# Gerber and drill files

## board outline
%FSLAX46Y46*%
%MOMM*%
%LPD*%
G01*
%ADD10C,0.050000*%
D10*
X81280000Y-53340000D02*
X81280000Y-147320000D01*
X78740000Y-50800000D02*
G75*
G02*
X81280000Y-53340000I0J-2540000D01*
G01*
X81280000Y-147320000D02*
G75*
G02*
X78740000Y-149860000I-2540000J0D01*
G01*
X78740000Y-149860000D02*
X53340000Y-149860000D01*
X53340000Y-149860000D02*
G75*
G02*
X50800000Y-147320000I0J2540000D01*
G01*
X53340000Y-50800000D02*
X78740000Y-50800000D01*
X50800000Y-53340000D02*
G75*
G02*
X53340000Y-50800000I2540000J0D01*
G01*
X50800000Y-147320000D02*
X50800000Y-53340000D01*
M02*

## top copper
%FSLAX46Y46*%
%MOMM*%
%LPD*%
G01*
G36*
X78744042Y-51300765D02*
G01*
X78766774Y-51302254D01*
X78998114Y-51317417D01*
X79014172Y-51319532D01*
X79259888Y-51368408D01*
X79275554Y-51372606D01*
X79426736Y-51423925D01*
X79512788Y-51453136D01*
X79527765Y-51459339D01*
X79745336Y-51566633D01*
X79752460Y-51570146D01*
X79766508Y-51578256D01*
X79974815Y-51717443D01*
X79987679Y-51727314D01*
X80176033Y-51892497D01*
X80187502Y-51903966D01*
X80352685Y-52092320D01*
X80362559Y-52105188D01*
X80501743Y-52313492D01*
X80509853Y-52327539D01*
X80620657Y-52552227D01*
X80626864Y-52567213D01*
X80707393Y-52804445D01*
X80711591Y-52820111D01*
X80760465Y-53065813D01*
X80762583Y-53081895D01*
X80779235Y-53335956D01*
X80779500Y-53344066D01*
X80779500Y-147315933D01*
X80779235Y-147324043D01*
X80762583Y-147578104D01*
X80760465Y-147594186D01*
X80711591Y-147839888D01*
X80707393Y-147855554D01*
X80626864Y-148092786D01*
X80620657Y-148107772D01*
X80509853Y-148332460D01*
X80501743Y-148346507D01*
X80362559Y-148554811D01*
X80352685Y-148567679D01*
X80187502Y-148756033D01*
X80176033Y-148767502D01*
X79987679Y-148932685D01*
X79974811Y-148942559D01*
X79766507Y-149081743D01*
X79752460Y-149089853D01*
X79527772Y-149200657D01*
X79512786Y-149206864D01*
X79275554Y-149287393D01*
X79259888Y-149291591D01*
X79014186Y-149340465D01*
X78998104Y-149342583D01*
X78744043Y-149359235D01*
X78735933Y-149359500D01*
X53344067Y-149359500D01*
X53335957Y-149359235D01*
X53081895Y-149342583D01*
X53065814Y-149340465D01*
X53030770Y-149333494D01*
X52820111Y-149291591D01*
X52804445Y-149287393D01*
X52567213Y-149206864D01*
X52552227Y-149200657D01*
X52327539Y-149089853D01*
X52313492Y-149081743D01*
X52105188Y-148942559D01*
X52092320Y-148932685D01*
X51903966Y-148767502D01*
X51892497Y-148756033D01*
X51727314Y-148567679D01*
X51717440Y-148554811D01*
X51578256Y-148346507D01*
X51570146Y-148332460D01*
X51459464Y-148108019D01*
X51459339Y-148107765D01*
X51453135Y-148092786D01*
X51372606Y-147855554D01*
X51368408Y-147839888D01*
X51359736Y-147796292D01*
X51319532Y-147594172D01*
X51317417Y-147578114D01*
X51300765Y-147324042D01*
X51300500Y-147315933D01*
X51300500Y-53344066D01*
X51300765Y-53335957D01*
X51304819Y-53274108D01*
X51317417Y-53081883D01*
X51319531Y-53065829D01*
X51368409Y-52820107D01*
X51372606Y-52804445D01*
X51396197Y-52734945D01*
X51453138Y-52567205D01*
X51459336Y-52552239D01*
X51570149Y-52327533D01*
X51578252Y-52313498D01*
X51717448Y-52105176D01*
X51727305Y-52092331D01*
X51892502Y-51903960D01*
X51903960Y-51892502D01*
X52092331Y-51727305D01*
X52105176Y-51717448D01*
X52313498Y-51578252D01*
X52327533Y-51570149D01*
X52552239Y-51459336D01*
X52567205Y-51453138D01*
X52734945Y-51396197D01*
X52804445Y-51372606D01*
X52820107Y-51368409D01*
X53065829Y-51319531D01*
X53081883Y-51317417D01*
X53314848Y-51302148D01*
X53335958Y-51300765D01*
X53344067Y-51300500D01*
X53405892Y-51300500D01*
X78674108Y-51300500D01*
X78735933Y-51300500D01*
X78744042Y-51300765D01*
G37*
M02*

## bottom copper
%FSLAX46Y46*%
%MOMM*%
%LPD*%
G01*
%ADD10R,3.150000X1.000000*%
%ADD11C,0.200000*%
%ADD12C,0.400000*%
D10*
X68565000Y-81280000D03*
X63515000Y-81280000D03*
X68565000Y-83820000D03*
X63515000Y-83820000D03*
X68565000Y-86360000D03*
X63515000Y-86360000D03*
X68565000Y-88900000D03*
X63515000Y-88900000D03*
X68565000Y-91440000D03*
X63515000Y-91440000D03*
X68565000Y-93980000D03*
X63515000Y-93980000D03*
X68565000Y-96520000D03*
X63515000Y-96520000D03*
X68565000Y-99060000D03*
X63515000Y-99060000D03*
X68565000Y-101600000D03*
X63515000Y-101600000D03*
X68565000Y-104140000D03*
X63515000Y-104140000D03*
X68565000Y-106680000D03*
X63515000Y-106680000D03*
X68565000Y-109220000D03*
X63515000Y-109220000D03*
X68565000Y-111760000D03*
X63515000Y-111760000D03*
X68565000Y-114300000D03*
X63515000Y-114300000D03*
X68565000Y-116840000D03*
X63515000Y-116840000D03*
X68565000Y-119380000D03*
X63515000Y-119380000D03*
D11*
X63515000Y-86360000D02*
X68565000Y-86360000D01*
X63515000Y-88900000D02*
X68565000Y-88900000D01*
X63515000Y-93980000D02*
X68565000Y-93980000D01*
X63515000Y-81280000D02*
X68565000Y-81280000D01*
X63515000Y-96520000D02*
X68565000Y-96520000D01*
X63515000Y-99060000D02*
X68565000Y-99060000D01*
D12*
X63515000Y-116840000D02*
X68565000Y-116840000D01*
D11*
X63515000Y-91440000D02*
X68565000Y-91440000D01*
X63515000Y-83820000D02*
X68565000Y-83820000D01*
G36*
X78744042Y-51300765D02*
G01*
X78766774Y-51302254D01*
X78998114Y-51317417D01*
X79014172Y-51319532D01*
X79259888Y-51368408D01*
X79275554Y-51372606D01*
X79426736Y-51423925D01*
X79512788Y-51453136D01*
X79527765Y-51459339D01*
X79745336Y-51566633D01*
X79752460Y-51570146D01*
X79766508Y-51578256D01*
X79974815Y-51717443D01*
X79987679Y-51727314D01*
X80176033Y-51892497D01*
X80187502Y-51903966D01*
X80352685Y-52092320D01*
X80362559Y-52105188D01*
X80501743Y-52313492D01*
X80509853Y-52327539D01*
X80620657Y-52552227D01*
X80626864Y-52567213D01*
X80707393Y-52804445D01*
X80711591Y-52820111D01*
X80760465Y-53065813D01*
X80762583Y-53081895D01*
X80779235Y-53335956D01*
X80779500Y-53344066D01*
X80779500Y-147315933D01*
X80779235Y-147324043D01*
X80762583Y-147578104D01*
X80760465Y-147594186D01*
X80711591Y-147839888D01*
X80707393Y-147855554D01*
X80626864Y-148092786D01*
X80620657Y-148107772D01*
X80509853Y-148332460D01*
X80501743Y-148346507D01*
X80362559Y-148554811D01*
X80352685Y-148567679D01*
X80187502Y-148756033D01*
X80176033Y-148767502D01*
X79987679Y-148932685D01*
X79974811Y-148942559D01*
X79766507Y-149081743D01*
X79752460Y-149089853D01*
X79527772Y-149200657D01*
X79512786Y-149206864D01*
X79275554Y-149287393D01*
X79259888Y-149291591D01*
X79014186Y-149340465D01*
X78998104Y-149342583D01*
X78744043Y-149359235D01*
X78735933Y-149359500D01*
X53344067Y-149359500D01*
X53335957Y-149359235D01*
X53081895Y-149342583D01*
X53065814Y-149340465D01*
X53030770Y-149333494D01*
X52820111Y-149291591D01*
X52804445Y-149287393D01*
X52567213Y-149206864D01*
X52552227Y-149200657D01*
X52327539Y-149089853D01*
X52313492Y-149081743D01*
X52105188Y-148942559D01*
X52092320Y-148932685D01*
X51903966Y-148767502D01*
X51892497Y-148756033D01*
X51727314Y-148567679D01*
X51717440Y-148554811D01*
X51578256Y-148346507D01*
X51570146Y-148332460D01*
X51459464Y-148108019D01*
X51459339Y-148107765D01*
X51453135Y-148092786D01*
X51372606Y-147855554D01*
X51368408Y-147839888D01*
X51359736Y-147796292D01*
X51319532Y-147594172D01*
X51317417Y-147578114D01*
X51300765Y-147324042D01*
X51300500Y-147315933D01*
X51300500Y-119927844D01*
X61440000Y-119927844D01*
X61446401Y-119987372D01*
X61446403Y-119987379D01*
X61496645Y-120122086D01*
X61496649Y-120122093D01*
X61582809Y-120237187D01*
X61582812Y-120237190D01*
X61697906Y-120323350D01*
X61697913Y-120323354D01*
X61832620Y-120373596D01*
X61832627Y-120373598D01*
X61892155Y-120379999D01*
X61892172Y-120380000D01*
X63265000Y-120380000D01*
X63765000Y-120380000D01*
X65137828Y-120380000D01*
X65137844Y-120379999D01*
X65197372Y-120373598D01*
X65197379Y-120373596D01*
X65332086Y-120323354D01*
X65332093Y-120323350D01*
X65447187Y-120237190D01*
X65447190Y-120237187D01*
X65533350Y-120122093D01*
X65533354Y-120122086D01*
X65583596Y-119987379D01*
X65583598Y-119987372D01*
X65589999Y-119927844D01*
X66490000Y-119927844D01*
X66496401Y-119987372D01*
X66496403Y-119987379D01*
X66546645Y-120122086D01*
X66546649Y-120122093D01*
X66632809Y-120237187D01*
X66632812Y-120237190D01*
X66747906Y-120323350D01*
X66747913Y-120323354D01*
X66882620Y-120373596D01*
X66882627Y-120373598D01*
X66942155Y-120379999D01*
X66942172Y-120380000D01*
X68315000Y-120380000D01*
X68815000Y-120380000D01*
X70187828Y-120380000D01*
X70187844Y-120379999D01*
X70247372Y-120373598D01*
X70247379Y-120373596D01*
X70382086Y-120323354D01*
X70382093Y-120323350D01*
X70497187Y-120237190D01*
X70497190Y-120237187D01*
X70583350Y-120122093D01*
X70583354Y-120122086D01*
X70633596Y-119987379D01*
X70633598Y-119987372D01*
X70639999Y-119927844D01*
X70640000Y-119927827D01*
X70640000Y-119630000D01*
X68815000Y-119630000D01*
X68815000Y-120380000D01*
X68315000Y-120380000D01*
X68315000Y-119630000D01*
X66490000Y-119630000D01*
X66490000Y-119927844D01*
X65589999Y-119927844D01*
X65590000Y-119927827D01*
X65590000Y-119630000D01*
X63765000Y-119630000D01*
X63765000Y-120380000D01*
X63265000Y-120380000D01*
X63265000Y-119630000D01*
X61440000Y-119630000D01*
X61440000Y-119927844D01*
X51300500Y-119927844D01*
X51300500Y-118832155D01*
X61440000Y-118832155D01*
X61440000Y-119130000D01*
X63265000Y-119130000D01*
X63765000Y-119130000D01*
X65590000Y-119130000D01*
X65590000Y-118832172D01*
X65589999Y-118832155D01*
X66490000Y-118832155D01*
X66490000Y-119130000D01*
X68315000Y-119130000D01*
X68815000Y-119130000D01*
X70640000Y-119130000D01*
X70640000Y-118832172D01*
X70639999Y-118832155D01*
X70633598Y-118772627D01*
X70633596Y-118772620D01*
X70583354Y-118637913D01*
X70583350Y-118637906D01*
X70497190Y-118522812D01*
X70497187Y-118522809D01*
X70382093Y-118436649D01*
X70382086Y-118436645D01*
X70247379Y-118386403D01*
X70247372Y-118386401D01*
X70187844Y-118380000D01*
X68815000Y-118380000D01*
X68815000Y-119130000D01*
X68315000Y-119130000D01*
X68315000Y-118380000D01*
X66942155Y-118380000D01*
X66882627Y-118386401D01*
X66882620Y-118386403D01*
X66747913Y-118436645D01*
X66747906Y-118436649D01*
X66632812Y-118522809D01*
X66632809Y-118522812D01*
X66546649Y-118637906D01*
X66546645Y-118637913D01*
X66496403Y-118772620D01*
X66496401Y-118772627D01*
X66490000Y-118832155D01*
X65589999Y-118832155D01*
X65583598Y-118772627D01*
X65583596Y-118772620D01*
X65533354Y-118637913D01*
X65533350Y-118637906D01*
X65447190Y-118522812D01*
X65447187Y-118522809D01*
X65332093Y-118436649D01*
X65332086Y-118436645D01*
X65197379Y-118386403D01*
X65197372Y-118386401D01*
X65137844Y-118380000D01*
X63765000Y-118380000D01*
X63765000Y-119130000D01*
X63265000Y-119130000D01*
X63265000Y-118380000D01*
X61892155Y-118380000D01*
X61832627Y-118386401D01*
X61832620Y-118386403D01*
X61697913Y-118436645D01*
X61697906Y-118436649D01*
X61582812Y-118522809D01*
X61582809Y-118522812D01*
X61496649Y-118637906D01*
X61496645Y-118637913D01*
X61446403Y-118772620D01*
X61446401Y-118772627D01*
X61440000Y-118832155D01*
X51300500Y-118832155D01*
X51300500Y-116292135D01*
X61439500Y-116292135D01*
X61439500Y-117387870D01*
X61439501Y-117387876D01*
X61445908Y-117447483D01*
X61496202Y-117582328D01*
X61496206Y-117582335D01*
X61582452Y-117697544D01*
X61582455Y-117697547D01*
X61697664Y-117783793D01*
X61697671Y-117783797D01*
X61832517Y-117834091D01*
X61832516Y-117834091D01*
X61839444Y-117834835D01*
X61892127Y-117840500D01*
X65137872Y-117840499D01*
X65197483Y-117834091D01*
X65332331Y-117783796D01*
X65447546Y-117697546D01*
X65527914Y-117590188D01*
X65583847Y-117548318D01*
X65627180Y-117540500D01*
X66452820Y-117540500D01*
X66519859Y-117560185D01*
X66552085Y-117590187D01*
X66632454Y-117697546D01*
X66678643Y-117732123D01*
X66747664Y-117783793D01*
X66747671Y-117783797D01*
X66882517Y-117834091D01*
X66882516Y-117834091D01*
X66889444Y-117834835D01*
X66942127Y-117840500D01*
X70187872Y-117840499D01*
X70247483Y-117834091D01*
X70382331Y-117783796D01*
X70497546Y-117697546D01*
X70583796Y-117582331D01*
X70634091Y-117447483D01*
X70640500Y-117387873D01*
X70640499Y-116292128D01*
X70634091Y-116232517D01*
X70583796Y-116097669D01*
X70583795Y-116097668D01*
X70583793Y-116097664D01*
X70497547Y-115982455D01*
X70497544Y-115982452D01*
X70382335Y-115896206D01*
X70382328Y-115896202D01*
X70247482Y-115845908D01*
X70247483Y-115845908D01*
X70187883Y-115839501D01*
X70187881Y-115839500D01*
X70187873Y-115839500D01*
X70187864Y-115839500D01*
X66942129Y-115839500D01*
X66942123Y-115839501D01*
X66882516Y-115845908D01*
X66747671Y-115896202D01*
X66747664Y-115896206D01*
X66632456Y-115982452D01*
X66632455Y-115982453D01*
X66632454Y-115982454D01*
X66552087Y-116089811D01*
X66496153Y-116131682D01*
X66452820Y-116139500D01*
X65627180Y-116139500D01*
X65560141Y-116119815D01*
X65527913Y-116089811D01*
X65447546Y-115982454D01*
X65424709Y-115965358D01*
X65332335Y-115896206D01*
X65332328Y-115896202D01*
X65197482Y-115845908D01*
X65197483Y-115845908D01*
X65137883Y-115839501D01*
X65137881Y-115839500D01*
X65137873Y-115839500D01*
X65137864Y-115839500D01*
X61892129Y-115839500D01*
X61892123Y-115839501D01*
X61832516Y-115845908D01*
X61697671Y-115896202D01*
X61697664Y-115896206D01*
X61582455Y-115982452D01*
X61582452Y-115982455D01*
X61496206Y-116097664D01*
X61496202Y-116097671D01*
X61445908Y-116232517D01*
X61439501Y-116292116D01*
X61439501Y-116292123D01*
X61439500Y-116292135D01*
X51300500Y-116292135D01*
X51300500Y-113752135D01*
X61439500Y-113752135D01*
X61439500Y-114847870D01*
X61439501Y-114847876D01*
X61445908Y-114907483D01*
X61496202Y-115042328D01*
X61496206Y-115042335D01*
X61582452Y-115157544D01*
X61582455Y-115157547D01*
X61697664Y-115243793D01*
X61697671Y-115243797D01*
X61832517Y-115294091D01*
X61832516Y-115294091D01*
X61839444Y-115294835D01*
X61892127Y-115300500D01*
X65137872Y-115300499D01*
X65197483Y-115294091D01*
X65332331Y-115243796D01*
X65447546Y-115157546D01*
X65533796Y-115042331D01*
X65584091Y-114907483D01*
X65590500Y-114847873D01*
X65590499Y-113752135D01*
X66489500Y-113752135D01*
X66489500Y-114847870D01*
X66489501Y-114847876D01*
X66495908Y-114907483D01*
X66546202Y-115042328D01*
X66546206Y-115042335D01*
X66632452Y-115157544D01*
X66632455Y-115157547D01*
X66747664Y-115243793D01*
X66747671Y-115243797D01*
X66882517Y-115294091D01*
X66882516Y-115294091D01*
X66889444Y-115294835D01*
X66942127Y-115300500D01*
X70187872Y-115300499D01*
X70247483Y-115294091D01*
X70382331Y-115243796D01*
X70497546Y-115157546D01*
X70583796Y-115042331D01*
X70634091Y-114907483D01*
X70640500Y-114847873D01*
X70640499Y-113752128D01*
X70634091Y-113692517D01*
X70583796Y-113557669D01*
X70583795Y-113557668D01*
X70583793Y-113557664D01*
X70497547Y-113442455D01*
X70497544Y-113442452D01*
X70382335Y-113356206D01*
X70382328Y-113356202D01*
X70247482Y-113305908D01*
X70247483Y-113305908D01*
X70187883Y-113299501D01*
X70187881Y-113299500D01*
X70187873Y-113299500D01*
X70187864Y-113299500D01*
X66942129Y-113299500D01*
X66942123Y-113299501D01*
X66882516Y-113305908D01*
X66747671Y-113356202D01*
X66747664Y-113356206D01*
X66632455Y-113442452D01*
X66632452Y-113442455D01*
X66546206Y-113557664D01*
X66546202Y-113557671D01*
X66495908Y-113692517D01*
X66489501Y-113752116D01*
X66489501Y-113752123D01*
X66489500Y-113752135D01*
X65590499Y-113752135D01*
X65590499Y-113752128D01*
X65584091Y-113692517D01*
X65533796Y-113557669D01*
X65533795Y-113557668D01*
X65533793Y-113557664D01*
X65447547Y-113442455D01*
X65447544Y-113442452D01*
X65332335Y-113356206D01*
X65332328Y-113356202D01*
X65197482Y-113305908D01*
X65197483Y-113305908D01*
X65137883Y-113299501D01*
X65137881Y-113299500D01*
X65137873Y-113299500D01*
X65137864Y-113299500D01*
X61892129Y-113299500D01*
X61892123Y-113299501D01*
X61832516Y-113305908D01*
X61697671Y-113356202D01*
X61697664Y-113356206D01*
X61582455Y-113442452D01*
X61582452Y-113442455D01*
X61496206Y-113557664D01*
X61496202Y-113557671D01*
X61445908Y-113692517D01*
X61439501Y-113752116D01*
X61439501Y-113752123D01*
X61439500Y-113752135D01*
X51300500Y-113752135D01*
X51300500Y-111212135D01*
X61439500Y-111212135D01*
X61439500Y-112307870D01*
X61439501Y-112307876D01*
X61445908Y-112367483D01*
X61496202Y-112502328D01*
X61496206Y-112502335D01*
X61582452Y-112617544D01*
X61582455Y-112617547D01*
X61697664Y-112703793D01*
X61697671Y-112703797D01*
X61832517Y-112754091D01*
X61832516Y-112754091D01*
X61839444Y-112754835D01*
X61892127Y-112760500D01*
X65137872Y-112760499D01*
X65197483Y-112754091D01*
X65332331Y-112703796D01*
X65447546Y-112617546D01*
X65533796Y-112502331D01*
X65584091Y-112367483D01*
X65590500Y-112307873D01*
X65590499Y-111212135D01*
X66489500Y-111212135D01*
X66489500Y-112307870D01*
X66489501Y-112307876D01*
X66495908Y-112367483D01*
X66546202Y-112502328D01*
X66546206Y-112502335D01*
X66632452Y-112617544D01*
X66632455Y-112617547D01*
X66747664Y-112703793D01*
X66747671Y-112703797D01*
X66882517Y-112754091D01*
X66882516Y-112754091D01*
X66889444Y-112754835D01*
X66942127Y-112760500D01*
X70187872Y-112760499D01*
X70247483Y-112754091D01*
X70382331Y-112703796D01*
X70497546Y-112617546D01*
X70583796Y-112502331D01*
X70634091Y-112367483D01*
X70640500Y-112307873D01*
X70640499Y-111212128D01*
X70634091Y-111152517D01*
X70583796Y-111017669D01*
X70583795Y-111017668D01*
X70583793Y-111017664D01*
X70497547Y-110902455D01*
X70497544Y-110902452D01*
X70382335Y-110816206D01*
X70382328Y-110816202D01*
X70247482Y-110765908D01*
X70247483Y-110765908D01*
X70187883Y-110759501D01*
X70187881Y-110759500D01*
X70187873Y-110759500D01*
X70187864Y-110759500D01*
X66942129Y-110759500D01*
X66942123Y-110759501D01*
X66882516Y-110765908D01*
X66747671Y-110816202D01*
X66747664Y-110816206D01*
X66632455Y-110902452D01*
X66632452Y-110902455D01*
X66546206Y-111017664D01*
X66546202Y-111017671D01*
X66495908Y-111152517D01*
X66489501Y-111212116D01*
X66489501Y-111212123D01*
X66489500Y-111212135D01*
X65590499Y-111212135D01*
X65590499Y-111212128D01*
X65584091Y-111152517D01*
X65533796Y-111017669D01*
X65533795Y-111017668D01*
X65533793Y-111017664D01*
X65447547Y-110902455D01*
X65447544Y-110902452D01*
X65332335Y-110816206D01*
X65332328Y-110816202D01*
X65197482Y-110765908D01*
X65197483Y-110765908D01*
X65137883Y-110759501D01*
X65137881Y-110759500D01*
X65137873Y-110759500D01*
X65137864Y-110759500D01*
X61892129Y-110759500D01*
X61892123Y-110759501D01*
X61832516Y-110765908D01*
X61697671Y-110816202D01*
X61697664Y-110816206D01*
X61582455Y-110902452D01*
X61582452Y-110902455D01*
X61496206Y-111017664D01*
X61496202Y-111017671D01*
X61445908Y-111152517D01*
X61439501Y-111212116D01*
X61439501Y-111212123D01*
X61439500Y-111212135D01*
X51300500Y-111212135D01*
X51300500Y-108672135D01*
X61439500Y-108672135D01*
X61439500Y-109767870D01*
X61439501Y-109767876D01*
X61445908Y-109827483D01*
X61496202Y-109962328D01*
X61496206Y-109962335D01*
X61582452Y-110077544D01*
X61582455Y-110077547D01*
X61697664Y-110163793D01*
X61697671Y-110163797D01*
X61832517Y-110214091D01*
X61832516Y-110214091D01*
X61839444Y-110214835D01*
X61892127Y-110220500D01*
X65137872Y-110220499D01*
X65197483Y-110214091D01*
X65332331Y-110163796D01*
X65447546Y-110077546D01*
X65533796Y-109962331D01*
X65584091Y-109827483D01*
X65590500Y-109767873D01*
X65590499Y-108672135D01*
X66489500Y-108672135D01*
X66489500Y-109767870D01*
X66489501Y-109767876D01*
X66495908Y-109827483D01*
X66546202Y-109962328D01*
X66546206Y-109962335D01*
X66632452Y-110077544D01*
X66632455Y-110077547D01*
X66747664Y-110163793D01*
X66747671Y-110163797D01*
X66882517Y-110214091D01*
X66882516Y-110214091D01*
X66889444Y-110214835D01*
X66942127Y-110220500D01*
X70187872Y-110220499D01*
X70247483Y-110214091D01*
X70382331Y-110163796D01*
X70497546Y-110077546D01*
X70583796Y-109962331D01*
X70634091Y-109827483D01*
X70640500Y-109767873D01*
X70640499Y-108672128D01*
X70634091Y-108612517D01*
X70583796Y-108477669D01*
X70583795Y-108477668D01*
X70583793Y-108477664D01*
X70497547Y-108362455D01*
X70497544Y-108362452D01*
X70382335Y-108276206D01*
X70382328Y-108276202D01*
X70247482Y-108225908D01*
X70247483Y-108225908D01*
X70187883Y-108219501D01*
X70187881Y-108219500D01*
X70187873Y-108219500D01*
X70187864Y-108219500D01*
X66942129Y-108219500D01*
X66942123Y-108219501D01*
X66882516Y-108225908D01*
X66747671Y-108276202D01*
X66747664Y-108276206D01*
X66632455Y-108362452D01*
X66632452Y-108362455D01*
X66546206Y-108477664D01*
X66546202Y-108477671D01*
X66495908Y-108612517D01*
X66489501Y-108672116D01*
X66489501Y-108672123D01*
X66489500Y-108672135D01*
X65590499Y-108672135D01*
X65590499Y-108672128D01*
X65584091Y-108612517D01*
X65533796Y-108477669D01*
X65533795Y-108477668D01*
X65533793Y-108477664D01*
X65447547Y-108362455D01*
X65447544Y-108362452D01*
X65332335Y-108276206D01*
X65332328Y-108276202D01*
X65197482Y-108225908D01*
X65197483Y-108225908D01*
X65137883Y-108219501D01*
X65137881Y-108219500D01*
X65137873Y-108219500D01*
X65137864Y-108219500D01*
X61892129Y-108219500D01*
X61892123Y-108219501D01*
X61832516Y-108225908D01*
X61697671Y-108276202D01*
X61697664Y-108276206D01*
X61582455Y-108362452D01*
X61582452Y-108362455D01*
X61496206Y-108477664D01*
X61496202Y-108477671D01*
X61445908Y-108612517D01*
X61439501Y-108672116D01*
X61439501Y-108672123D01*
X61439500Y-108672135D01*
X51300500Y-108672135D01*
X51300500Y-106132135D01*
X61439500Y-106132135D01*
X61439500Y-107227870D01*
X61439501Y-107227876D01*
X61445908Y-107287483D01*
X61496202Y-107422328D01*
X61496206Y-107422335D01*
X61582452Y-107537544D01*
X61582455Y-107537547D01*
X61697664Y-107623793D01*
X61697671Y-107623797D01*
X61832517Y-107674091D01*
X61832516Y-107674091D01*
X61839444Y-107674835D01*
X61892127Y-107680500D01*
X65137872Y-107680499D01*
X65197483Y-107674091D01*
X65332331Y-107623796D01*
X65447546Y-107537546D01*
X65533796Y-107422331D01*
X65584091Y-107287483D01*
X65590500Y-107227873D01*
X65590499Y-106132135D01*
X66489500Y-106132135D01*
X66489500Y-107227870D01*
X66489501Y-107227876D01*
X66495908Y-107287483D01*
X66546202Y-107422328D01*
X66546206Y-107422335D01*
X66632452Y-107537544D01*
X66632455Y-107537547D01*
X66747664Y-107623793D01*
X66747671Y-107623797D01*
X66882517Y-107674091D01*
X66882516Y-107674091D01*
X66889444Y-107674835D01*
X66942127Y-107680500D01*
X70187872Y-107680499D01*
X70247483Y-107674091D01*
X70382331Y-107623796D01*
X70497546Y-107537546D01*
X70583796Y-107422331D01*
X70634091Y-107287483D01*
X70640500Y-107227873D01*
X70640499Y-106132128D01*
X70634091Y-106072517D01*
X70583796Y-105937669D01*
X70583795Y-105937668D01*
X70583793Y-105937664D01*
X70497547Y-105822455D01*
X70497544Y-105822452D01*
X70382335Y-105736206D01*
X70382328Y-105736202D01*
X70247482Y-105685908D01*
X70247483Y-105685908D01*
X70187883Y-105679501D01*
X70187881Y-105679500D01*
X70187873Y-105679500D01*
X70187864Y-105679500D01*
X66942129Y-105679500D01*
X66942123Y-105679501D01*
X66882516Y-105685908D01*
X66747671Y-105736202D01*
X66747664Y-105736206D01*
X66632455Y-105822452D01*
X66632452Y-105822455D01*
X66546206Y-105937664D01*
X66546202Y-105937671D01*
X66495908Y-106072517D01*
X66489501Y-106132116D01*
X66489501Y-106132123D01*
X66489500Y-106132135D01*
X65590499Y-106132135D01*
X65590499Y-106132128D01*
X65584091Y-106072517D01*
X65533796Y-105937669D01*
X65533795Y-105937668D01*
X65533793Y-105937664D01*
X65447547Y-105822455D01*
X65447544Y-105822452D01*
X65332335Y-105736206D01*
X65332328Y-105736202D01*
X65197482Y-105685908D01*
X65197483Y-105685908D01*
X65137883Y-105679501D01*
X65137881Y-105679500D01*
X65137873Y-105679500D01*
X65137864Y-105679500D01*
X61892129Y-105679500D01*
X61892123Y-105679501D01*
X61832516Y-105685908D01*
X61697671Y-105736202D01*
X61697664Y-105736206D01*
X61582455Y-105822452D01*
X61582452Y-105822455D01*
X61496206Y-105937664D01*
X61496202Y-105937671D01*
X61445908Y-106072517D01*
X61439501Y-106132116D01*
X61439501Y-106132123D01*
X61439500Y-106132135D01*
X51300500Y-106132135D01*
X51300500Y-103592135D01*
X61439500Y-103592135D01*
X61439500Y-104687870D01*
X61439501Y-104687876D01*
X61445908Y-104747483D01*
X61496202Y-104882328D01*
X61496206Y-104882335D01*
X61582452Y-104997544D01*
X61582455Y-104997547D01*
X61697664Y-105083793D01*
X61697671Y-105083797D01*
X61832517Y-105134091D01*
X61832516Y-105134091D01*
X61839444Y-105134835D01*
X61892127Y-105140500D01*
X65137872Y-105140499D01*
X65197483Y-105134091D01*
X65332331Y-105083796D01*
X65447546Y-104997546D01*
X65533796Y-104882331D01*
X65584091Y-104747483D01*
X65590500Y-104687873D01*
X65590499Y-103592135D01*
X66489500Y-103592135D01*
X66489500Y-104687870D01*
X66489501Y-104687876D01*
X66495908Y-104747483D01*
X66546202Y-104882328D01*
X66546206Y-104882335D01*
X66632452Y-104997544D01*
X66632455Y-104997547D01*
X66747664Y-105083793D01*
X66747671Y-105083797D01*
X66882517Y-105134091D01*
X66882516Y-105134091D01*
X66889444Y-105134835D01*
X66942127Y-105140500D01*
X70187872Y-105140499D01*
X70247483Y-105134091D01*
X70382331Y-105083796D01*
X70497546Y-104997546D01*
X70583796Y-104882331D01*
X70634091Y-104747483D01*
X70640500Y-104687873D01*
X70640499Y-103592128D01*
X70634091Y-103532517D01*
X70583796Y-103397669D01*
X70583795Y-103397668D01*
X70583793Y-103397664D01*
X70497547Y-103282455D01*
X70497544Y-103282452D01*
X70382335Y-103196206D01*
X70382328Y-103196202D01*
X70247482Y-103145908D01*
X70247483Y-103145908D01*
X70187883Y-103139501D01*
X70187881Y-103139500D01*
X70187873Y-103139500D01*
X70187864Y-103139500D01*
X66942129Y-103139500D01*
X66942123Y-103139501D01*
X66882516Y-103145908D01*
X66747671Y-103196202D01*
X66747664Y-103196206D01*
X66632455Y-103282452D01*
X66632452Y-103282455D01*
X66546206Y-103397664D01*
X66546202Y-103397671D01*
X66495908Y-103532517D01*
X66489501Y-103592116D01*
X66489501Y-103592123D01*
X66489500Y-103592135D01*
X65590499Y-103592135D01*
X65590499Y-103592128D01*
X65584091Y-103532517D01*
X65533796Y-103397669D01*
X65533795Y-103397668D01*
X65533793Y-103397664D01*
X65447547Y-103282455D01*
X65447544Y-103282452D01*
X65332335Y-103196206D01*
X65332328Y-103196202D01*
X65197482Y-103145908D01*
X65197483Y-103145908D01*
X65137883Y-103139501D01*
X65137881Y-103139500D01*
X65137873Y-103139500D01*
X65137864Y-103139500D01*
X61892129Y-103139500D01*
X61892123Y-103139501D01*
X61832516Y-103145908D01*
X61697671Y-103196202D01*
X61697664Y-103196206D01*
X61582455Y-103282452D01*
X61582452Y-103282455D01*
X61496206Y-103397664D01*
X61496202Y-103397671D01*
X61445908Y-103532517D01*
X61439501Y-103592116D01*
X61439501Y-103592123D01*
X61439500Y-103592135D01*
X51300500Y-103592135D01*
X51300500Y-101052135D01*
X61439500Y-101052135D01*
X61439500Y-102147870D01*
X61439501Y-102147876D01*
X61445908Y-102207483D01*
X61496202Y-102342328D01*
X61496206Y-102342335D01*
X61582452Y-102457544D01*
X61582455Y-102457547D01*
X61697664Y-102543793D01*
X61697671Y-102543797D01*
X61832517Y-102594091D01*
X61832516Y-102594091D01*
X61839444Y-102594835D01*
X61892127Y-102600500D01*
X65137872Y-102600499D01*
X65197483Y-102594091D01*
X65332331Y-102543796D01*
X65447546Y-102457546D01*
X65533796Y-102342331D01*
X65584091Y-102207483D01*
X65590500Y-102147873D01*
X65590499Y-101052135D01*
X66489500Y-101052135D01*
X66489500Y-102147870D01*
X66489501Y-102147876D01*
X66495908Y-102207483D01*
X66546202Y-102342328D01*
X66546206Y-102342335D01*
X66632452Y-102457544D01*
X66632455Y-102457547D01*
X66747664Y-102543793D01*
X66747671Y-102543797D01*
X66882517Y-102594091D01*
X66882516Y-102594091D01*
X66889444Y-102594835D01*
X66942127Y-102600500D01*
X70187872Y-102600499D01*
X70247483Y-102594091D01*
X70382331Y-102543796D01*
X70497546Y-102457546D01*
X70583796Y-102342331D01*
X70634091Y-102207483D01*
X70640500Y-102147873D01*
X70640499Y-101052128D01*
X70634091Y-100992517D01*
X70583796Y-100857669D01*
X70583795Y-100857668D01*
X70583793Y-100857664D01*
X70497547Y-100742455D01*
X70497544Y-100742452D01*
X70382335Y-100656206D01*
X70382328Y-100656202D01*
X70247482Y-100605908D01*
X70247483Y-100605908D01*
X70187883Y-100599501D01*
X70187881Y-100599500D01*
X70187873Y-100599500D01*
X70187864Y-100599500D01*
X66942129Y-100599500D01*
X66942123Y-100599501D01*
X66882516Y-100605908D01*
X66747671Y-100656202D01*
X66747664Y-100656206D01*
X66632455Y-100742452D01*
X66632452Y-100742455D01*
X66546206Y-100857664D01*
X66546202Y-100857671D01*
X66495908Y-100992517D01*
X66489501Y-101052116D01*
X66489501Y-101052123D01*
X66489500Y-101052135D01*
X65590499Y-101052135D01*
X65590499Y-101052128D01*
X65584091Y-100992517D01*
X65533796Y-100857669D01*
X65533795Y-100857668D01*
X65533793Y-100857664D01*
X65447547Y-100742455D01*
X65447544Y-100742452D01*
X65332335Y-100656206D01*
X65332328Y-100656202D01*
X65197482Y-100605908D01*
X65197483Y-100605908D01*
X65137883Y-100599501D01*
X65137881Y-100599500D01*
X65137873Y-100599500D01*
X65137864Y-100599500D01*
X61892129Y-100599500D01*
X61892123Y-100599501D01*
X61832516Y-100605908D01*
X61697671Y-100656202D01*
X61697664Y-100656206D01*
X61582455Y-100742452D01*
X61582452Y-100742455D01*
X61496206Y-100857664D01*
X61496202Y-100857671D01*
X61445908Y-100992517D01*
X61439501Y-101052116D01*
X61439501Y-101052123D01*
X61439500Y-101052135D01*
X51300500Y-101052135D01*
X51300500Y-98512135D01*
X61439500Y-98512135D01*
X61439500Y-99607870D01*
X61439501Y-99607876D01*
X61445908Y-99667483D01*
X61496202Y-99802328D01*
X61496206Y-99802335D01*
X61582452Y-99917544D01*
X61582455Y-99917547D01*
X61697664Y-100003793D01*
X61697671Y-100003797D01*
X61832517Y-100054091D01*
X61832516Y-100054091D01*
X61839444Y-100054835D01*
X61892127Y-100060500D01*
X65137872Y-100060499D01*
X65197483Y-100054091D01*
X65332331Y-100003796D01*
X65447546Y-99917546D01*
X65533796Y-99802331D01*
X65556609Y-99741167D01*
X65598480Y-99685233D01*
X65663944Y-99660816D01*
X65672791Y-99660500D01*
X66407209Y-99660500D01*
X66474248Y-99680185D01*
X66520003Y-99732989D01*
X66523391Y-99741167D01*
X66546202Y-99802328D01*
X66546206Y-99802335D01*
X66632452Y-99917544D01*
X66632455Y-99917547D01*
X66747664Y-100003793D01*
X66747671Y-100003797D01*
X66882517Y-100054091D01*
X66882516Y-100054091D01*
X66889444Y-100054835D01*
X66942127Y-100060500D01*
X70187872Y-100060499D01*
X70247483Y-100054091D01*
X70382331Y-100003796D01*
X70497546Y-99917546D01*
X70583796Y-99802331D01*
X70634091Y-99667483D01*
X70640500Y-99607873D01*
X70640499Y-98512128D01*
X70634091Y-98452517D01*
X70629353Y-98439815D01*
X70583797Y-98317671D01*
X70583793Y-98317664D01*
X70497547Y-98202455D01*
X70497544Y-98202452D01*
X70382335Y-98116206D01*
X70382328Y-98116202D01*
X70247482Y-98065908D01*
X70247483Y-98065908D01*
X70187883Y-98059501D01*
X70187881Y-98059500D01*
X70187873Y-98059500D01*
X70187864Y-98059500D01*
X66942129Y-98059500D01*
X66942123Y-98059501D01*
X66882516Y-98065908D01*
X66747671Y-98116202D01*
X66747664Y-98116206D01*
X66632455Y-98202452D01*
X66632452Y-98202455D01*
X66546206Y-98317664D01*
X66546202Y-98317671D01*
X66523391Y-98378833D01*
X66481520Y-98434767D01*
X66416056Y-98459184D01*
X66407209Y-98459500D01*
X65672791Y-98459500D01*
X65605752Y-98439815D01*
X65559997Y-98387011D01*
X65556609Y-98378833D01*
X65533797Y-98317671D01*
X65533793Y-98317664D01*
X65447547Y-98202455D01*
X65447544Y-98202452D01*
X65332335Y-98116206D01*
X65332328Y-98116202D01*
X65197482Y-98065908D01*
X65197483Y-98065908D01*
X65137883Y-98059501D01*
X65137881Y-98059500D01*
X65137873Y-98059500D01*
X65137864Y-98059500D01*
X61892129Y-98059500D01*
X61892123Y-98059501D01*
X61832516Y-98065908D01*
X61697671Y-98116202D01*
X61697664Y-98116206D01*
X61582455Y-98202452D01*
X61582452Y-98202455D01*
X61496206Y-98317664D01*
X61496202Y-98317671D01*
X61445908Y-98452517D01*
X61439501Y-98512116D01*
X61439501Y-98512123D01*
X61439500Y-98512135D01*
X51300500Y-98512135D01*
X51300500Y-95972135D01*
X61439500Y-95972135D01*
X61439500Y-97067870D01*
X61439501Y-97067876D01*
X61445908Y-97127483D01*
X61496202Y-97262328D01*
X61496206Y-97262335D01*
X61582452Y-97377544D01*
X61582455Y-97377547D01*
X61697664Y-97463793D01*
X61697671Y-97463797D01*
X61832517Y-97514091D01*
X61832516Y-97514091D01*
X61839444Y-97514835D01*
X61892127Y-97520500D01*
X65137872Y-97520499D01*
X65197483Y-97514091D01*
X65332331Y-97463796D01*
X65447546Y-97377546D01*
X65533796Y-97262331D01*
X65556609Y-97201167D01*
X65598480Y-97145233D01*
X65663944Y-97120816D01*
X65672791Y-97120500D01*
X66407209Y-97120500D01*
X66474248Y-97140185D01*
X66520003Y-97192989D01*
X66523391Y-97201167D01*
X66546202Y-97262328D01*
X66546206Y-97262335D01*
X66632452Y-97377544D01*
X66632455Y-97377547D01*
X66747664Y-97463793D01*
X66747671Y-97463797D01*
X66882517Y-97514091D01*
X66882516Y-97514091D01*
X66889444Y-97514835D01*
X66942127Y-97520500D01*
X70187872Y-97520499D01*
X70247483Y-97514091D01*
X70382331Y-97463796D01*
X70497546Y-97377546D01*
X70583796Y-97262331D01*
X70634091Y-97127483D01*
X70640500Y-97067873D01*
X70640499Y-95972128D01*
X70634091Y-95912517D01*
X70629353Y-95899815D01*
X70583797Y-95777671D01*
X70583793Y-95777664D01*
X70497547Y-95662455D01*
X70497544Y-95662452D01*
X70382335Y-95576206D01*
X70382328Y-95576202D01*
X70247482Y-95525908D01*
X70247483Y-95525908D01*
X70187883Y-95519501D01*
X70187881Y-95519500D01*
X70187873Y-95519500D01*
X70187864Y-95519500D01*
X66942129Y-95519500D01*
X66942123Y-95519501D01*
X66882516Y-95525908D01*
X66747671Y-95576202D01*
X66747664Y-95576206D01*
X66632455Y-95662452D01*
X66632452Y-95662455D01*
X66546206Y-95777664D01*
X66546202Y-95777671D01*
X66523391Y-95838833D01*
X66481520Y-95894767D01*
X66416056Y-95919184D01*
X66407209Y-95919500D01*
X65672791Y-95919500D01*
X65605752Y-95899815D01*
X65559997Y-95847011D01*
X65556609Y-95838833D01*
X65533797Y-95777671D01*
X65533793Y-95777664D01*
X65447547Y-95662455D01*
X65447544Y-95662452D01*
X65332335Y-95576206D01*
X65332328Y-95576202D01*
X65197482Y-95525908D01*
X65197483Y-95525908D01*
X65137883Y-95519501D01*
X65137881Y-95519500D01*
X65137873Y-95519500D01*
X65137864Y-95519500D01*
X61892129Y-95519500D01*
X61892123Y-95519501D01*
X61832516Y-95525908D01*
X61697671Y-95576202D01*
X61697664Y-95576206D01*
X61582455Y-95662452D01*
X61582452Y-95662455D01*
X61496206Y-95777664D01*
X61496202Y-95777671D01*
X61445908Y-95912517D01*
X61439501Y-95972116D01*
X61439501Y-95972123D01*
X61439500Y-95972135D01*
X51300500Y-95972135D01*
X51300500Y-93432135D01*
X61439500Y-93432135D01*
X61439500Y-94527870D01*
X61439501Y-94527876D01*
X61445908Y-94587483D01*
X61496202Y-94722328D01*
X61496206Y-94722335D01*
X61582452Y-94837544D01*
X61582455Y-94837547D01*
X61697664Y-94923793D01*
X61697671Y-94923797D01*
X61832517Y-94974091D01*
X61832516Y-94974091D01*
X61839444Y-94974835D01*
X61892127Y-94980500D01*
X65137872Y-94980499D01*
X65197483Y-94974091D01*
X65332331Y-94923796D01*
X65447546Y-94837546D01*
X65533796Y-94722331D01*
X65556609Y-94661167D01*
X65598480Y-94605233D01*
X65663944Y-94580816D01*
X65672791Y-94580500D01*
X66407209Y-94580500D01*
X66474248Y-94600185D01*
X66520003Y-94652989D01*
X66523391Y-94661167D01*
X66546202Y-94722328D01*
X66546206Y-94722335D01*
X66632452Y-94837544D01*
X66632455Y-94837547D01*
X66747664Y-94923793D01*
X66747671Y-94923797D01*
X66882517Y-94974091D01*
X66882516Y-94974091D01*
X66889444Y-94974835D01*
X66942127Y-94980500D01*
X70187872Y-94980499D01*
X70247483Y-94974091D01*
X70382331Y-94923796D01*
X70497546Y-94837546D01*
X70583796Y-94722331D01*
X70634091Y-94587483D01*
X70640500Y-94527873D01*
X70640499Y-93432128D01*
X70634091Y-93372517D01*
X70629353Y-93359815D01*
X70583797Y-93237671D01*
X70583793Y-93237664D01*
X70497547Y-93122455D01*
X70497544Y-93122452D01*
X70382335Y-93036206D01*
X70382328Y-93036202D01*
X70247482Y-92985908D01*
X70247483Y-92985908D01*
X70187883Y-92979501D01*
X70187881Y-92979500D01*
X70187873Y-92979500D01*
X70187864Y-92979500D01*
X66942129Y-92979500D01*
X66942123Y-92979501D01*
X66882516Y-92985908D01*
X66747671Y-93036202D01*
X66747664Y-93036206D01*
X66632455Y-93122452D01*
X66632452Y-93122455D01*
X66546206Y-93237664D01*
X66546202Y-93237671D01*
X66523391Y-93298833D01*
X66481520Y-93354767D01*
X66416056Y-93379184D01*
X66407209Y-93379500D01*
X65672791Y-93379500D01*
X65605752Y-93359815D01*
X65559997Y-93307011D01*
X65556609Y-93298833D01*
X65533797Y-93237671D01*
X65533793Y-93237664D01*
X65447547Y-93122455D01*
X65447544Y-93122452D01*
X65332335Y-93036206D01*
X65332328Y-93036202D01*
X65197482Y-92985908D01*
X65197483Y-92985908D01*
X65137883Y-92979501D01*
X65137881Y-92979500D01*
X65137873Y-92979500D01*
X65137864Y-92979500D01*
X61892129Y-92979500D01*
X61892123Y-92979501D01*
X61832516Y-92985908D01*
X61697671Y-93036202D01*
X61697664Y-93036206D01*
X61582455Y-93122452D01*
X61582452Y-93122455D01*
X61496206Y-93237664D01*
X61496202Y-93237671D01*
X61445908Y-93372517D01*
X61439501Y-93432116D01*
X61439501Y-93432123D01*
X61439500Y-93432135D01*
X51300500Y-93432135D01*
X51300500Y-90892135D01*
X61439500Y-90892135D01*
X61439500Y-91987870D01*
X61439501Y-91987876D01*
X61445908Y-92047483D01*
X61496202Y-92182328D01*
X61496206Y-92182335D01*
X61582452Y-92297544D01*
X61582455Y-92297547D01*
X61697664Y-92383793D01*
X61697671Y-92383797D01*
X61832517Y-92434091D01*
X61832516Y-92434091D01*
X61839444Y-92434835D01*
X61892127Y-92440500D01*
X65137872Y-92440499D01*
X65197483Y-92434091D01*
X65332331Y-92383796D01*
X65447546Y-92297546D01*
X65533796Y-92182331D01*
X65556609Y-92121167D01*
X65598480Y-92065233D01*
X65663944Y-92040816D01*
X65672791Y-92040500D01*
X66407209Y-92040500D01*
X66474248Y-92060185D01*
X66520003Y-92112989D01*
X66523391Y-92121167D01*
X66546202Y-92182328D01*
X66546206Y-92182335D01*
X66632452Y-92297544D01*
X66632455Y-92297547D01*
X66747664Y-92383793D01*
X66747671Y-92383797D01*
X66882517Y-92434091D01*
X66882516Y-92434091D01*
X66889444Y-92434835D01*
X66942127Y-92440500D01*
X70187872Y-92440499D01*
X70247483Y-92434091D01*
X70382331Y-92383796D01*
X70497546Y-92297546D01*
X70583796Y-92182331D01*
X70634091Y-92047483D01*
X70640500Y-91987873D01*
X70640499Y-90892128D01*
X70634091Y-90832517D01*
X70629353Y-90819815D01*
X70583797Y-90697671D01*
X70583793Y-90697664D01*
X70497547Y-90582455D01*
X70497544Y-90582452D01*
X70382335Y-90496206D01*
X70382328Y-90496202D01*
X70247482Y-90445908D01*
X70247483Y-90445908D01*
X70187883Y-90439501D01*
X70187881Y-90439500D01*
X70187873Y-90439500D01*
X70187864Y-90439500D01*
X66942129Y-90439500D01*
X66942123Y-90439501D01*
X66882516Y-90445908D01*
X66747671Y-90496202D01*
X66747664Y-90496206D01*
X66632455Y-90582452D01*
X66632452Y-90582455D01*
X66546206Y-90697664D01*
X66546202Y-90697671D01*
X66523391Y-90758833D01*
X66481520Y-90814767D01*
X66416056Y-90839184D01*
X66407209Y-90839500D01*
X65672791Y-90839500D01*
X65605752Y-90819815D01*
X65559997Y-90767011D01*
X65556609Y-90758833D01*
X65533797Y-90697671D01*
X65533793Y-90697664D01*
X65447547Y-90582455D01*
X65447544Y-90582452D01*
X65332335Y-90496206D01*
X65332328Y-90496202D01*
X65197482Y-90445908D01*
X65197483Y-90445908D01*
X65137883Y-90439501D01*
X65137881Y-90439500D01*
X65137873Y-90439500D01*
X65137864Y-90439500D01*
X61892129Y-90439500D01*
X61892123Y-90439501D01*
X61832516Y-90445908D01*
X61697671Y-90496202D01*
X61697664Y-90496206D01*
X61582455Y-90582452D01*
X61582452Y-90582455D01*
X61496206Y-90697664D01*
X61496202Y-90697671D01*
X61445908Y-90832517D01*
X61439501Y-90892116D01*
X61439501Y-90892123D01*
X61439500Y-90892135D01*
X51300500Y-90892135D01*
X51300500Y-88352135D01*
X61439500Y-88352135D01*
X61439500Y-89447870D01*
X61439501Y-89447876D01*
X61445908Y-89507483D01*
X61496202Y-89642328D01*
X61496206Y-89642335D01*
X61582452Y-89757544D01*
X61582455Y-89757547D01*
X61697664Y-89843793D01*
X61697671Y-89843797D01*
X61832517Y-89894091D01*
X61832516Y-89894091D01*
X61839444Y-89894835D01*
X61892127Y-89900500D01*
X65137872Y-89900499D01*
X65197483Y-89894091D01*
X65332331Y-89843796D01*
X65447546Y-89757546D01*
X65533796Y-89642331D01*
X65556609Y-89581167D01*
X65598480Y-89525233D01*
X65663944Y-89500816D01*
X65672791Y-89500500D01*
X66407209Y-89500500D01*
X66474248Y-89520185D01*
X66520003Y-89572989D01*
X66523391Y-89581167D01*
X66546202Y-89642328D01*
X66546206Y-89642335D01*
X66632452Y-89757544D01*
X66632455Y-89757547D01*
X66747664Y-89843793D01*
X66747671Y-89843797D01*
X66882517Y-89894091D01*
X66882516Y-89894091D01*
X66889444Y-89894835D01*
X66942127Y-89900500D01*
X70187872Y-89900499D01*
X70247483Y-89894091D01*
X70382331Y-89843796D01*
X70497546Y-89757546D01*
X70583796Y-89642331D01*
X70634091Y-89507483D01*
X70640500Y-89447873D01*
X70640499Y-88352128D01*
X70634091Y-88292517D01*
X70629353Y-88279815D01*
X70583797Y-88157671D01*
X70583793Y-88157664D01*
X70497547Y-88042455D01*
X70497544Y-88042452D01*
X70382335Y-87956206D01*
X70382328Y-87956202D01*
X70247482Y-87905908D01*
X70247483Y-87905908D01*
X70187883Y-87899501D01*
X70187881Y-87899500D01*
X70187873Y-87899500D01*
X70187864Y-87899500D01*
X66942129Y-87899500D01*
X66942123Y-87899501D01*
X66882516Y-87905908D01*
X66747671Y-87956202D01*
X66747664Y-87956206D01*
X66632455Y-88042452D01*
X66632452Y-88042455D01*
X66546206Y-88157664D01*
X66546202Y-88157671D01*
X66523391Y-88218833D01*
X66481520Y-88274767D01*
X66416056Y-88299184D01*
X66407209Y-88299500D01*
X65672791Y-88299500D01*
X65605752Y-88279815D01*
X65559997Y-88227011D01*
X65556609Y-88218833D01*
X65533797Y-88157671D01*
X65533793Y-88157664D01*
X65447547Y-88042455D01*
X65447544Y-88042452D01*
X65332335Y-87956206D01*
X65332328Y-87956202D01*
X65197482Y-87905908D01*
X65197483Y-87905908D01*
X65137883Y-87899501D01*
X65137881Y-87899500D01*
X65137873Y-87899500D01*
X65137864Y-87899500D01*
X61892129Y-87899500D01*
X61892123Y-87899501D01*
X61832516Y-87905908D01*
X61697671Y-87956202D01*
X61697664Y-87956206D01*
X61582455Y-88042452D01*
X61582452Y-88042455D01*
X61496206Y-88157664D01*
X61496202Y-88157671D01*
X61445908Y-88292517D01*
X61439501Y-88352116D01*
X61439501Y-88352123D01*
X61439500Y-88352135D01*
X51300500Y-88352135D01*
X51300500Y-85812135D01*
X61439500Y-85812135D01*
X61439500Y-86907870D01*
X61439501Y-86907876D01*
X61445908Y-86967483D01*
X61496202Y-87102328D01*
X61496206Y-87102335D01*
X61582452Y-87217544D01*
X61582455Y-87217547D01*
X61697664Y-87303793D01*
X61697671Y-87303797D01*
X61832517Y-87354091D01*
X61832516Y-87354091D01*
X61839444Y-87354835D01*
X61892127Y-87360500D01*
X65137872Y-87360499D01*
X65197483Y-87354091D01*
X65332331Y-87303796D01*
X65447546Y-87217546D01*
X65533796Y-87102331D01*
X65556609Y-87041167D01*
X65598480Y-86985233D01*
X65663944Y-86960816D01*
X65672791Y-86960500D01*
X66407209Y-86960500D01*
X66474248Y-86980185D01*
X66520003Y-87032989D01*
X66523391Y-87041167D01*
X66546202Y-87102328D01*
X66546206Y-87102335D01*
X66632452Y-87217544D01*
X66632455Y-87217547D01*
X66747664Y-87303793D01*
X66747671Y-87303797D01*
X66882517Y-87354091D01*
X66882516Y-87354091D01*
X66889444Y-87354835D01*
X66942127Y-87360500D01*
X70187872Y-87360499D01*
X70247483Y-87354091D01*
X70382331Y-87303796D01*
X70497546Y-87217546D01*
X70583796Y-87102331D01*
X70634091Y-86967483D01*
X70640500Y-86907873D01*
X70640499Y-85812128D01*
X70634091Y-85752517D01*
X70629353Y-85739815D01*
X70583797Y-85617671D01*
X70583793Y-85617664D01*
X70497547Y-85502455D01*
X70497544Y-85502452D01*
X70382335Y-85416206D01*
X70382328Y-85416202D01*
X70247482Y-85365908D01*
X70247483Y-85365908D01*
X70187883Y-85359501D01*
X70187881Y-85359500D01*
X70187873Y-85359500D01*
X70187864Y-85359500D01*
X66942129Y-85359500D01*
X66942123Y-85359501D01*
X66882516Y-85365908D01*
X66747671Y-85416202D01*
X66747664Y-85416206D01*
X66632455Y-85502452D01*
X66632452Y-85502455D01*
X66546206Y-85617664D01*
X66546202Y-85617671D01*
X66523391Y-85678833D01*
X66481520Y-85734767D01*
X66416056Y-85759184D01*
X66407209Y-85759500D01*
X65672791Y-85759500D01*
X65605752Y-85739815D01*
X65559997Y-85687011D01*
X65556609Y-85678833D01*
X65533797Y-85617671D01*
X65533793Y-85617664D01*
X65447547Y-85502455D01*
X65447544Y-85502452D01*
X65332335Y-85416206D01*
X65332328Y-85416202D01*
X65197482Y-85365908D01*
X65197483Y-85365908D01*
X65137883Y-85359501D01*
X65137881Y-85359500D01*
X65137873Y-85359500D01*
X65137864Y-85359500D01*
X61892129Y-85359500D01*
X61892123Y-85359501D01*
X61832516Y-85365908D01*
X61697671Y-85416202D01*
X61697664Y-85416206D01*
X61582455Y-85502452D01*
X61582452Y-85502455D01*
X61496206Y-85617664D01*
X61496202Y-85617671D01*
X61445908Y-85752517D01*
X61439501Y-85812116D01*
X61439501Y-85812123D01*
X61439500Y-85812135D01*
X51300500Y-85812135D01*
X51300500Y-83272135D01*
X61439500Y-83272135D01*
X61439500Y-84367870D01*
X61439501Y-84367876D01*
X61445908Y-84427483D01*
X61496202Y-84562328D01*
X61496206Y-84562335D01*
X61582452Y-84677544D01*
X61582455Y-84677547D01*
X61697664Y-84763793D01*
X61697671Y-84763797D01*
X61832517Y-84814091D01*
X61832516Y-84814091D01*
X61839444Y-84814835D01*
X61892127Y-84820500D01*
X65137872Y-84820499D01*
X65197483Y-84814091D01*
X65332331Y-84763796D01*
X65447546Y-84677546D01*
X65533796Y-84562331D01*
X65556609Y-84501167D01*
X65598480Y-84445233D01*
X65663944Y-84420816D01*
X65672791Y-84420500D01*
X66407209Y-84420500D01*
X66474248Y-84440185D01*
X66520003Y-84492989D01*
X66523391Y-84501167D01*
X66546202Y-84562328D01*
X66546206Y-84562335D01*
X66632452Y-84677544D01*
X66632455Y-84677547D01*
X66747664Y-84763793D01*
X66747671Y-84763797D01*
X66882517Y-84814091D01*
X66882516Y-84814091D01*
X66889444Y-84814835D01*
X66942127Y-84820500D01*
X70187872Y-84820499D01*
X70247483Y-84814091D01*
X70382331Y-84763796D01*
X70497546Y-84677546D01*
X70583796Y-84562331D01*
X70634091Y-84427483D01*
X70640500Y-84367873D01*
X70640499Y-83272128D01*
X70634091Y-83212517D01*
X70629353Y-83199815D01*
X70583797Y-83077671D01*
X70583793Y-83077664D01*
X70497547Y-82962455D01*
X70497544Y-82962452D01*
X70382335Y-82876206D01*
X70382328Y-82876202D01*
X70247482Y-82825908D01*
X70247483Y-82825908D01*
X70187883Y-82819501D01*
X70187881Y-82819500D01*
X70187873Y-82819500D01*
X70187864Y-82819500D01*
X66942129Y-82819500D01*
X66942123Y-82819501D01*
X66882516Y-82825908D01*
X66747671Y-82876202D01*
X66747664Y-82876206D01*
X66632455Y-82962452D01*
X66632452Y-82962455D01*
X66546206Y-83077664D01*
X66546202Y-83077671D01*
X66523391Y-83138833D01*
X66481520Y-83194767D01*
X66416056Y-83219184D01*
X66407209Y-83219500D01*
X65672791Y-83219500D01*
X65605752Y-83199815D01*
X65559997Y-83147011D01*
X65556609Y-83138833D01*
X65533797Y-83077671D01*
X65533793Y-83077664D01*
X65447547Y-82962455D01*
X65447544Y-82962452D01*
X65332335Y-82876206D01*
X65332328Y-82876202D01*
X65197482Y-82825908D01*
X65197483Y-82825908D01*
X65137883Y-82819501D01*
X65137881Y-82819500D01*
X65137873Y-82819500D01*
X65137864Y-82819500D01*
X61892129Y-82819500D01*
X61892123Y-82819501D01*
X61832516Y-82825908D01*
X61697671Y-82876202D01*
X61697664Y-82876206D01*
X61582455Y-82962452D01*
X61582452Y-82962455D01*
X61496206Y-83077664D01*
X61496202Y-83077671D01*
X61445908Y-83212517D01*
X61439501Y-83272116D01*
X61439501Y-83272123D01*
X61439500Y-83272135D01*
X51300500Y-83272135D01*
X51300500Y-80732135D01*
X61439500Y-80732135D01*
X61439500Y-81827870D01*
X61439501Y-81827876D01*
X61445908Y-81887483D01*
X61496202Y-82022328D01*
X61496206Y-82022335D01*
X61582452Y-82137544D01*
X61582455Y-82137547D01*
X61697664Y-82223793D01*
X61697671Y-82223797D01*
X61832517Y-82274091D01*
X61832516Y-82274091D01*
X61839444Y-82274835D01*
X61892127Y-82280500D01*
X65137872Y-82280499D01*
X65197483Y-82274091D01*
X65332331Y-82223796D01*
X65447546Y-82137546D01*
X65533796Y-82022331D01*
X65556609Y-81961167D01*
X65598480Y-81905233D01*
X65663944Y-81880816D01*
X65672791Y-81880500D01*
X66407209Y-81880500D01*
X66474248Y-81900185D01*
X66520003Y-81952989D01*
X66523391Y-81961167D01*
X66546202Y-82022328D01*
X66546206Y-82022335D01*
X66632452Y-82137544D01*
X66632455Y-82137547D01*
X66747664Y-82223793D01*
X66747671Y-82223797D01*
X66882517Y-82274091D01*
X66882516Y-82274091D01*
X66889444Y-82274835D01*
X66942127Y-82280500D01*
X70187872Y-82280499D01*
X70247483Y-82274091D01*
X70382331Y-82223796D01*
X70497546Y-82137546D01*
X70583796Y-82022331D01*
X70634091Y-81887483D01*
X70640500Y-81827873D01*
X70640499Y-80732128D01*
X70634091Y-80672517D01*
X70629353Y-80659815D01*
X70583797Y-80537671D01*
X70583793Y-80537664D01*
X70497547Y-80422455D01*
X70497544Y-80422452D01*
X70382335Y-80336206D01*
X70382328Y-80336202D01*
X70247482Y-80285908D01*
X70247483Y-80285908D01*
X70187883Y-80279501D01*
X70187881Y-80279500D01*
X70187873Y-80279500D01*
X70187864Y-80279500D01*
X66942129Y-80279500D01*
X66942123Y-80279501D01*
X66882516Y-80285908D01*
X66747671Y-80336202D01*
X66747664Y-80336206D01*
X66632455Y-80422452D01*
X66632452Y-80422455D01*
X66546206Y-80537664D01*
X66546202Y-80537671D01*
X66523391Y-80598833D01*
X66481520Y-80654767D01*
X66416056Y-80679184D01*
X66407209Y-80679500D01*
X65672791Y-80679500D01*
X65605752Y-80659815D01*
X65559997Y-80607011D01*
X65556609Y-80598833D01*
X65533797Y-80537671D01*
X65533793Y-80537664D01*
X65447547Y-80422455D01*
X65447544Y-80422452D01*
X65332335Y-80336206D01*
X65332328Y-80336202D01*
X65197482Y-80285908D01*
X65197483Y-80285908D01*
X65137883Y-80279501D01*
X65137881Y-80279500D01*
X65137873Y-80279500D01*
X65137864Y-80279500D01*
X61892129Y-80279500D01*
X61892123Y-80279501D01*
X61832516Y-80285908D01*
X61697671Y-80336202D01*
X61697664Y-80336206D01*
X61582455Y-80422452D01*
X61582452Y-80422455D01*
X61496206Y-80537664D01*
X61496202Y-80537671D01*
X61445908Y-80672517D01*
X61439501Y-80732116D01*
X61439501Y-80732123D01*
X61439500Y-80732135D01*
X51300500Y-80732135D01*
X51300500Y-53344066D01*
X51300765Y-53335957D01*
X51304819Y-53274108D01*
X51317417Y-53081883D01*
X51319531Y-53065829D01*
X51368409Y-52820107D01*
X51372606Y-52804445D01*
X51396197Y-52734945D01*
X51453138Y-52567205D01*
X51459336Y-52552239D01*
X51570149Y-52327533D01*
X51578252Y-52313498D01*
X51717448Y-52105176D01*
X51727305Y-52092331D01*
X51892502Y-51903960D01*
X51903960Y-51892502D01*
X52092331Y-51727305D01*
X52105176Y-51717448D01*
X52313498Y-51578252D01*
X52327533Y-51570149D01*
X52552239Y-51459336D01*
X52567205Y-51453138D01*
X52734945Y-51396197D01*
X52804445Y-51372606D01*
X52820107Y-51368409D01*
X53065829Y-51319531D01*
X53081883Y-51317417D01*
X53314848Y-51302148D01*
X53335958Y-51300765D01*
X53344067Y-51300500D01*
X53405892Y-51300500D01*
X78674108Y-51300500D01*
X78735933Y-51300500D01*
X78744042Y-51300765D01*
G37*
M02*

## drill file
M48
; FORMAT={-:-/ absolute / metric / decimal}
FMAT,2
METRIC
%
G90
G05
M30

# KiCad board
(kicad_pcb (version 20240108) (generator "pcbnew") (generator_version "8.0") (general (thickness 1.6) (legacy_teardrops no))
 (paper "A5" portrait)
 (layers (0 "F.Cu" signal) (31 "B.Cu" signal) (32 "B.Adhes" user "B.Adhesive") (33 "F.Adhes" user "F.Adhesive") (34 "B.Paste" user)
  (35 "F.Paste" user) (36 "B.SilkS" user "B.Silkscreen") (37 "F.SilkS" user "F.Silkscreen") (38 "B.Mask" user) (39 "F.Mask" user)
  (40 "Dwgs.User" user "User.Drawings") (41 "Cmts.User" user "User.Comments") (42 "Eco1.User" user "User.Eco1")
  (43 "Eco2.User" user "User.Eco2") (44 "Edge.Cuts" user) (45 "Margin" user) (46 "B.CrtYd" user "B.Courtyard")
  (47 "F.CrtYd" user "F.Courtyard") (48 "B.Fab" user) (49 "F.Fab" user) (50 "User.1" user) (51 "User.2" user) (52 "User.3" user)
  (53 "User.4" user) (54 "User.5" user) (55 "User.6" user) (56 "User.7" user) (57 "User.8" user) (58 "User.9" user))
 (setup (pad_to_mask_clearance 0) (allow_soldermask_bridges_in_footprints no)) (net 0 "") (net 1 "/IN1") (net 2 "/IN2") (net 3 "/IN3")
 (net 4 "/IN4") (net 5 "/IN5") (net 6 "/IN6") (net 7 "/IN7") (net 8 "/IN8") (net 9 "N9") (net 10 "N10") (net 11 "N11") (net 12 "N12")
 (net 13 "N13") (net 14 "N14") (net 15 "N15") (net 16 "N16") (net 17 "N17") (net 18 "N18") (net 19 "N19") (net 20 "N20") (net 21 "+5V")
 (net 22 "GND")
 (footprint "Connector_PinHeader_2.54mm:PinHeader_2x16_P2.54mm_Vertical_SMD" (layer "B.Cu") (at 66.04 100.33 180)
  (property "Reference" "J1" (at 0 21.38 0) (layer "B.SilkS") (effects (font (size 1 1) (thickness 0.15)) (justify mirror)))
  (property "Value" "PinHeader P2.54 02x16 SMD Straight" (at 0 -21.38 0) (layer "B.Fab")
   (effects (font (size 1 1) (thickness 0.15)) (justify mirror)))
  (pad "1" smd rect (at -2.525 19.05 180) (size 3.15 1) (layers "B.Cu" "B.Paste" "B.Mask") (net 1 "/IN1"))
  (pad "2" smd rect (at 2.525 19.05 180) (size 3.15 1) (layers "B.Cu" "B.Paste" "B.Mask") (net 1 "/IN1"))
  (pad "3" smd rect (at -2.525 16.51 180) (size 3.15 1) (layers "B.Cu" "B.Paste" "B.Mask") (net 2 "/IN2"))
  (pad "4" smd rect (at 2.525 16.51 180) (size 3.15 1) (layers "B.Cu" "B.Paste" "B.Mask") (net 2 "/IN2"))
  (pad "5" smd rect (at -2.525 13.97 180) (size 3.15 1) (layers "B.Cu" "B.Paste" "B.Mask") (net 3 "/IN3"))
  (pad "6" smd rect (at 2.525 13.97 180) (size 3.15 1) (layers "B.Cu" "B.Paste" "B.Mask") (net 3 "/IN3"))
  (pad "7" smd rect (at -2.525 11.43 180) (size 3.15 1) (layers "B.Cu" "B.Paste" "B.Mask") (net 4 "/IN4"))
  (pad "8" smd rect (at 2.525 11.43 180) (size 3.15 1) (layers "B.Cu" "B.Paste" "B.Mask") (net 4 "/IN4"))
  (pad "9" smd rect (at -2.525 8.89 180) (size 3.15 1) (layers "B.Cu" "B.Paste" "B.Mask") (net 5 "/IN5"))
  (pad "10" smd rect (at 2.525 8.89 180) (size 3.15 1) (layers "B.Cu" "B.Paste" "B.Mask") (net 5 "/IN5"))
  (pad "11" smd rect (at -2.525 6.35 180) (size 3.15 1) (layers "B.Cu" "B.Paste" "B.Mask") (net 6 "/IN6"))
  (pad "12" smd rect (at 2.525 6.35 180) (size 3.15 1) (layers "B.Cu" "B.Paste" "B.Mask") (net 6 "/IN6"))
  (pad "13" smd rect (at -2.525 3.81 180) (size 3.15 1) (layers "B.Cu" "B.Paste" "B.Mask") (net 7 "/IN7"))
  (pad "14" smd rect (at 2.525 3.81 180) (size 3.15 1) (layers "B.Cu" "B.Paste" "B.Mask") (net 7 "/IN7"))
  (pad "15" smd rect (at -2.525 1.27 180) (size 3.15 1) (layers "B.Cu" "B.Paste" "B.Mask") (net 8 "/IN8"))
  (pad "16" smd rect (at 2.525 1.27 180) (size 3.15 1) (layers "B.Cu" "B.Paste" "B.Mask") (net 8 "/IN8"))
  (pad "17" smd rect (at -2.525 -1.27 180) (size 3.15 1) (layers "B.Cu" "B.Paste" "B.Mask") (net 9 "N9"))
  (pad "18" smd rect (at 2.525 -1.27 180) (size 3.15 1) (layers "B.Cu" "B.Paste" "B.Mask") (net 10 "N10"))
  (pad "19" smd rect (at -2.525 -3.81 180) (size 3.15 1) (layers "B.Cu" "B.Paste" "B.Mask") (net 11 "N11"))
  (pad "20" smd rect (at 2.525 -3.81 180) (size 3.15 1) (layers "B.Cu" "B.Paste" "B.Mask") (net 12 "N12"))
  (pad "21" smd rect (at -2.525 -6.35 180) (size 3.15 1) (layers "B.Cu" "B.Paste" "B.Mask") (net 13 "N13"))
  (pad "22" smd rect (at 2.525 -6.35 180) (size 3.15 1) (layers "B.Cu" "B.Paste" "B.Mask") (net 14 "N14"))
  (pad "23" smd rect (at -2.525 -8.89 180) (size 3.15 1) (layers "B.Cu" "B.Paste" "B.Mask") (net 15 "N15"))
  (pad "24" smd rect (at 2.525 -8.89 180) (size 3.15 1) (layers "B.Cu" "B.Paste" "B.Mask") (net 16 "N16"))
  (pad "25" smd rect (at -2.525 -11.43 180) (size 3.15 1) (layers "B.Cu" "B.Paste" "B.Mask") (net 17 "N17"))
  (pad "26" smd rect (at 2.525 -11.43 180) (size 3.15 1) (layers "B.Cu" "B.Paste" "B.Mask") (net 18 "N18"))
  (pad "27" smd rect (at -2.525 -13.97 180) (size 3.15 1) (layers "B.Cu" "B.Paste" "B.Mask") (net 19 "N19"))
  (pad "28" smd rect (at 2.525 -13.97 180) (size 3.15 1) (layers "B.Cu" "B.Paste" "B.Mask") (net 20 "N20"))
  (pad "29" smd rect (at -2.525 -16.51 180) (size 3.15 1) (layers "B.Cu" "B.Paste" "B.Mask") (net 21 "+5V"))
  (pad "30" smd rect (at 2.525 -16.51 180) (size 3.15 1) (layers "B.Cu" "B.Paste" "B.Mask") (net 21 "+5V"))
  (pad "31" smd rect (at -2.525 -19.05 180) (size 3.15 1) (layers "B.Cu" "B.Paste" "B.Mask") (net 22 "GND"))
  (pad "32" smd rect (at 2.525 -19.05 180) (size 3.15 1) (layers "B.Cu" "B.Paste" "B.Mask") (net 22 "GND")))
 (gr_line (start 81.28 53.34) (end 81.28 147.32) (stroke (width 0.05) (type default)) (layer "Edge.Cuts"))
 (gr_arc (start 78.74 50.8) (mid 80.536051 51.543949) (end 81.28 53.34) (stroke (width 0.05) (type default)) (layer "Edge.Cuts"))
 (gr_arc (start 81.28 147.32) (mid 80.536051 149.116051) (end 78.74 149.86) (stroke (width 0.05) (type default)) (layer "Edge.Cuts"))
 (gr_line (start 78.74 149.86) (end 53.34 149.86) (stroke (width 0.05) (type default)) (layer "Edge.Cuts"))
 (gr_arc (start 53.34 149.86) (mid 51.543949 149.116051) (end 50.8 147.32) (stroke (width 0.05) (type default)) (layer "Edge.Cuts"))
 (gr_line (start 53.34 50.8) (end 78.74 50.8) (stroke (width 0.05) (type default)) (layer "Edge.Cuts"))
 (gr_arc (start 50.8 53.34) (mid 51.543949 51.543949) (end 53.34 50.8) (stroke (width 0.05) (type default)) (layer "Edge.Cuts"))
 (gr_line (start 50.8 147.32) (end 50.8 53.34) (stroke (width 0.05) (type default)) (layer "Edge.Cuts"))
 (segment (start 63.515 86.36) (end 68.565 86.36) (width 0.2) (layer "B.Cu") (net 3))
 (segment (start 63.515 88.9) (end 68.565 88.9) (width 0.2) (layer "B.Cu") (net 4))
 (segment (start 63.515 93.98) (end 68.565 93.98) (width 0.2) (layer "B.Cu") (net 6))
 (segment (start 63.515 81.28) (end 68.565 81.28) (width 0.2) (layer "B.Cu") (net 1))
 (segment (start 63.515 96.52) (end 68.565 96.52) (width 0.2) (layer "B.Cu") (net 7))
 (segment (start 63.515 99.06) (end 68.565 99.06) (width 0.2) (layer "B.Cu") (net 8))
 (segment (start 63.515 116.84) (end 68.565 116.84) (width 0.4) (layer "B.Cu") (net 21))
 (segment (start 63.515 91.44) (end 68.565 91.44) (width 0.2) (layer "B.Cu") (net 5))
 (segment (start 63.515 83.82) (end 68.565 83.82) (width 0.2) (layer "B.Cu") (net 2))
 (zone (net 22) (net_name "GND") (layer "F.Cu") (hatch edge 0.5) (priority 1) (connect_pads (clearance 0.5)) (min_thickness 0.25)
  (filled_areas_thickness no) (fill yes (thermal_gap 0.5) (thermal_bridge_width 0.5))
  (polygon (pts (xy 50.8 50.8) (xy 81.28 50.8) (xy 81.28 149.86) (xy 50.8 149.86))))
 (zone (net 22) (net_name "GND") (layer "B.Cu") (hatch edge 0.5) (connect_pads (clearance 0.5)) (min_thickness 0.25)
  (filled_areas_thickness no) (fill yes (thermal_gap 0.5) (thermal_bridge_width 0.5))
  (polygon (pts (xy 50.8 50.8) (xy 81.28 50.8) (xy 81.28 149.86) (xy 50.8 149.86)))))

